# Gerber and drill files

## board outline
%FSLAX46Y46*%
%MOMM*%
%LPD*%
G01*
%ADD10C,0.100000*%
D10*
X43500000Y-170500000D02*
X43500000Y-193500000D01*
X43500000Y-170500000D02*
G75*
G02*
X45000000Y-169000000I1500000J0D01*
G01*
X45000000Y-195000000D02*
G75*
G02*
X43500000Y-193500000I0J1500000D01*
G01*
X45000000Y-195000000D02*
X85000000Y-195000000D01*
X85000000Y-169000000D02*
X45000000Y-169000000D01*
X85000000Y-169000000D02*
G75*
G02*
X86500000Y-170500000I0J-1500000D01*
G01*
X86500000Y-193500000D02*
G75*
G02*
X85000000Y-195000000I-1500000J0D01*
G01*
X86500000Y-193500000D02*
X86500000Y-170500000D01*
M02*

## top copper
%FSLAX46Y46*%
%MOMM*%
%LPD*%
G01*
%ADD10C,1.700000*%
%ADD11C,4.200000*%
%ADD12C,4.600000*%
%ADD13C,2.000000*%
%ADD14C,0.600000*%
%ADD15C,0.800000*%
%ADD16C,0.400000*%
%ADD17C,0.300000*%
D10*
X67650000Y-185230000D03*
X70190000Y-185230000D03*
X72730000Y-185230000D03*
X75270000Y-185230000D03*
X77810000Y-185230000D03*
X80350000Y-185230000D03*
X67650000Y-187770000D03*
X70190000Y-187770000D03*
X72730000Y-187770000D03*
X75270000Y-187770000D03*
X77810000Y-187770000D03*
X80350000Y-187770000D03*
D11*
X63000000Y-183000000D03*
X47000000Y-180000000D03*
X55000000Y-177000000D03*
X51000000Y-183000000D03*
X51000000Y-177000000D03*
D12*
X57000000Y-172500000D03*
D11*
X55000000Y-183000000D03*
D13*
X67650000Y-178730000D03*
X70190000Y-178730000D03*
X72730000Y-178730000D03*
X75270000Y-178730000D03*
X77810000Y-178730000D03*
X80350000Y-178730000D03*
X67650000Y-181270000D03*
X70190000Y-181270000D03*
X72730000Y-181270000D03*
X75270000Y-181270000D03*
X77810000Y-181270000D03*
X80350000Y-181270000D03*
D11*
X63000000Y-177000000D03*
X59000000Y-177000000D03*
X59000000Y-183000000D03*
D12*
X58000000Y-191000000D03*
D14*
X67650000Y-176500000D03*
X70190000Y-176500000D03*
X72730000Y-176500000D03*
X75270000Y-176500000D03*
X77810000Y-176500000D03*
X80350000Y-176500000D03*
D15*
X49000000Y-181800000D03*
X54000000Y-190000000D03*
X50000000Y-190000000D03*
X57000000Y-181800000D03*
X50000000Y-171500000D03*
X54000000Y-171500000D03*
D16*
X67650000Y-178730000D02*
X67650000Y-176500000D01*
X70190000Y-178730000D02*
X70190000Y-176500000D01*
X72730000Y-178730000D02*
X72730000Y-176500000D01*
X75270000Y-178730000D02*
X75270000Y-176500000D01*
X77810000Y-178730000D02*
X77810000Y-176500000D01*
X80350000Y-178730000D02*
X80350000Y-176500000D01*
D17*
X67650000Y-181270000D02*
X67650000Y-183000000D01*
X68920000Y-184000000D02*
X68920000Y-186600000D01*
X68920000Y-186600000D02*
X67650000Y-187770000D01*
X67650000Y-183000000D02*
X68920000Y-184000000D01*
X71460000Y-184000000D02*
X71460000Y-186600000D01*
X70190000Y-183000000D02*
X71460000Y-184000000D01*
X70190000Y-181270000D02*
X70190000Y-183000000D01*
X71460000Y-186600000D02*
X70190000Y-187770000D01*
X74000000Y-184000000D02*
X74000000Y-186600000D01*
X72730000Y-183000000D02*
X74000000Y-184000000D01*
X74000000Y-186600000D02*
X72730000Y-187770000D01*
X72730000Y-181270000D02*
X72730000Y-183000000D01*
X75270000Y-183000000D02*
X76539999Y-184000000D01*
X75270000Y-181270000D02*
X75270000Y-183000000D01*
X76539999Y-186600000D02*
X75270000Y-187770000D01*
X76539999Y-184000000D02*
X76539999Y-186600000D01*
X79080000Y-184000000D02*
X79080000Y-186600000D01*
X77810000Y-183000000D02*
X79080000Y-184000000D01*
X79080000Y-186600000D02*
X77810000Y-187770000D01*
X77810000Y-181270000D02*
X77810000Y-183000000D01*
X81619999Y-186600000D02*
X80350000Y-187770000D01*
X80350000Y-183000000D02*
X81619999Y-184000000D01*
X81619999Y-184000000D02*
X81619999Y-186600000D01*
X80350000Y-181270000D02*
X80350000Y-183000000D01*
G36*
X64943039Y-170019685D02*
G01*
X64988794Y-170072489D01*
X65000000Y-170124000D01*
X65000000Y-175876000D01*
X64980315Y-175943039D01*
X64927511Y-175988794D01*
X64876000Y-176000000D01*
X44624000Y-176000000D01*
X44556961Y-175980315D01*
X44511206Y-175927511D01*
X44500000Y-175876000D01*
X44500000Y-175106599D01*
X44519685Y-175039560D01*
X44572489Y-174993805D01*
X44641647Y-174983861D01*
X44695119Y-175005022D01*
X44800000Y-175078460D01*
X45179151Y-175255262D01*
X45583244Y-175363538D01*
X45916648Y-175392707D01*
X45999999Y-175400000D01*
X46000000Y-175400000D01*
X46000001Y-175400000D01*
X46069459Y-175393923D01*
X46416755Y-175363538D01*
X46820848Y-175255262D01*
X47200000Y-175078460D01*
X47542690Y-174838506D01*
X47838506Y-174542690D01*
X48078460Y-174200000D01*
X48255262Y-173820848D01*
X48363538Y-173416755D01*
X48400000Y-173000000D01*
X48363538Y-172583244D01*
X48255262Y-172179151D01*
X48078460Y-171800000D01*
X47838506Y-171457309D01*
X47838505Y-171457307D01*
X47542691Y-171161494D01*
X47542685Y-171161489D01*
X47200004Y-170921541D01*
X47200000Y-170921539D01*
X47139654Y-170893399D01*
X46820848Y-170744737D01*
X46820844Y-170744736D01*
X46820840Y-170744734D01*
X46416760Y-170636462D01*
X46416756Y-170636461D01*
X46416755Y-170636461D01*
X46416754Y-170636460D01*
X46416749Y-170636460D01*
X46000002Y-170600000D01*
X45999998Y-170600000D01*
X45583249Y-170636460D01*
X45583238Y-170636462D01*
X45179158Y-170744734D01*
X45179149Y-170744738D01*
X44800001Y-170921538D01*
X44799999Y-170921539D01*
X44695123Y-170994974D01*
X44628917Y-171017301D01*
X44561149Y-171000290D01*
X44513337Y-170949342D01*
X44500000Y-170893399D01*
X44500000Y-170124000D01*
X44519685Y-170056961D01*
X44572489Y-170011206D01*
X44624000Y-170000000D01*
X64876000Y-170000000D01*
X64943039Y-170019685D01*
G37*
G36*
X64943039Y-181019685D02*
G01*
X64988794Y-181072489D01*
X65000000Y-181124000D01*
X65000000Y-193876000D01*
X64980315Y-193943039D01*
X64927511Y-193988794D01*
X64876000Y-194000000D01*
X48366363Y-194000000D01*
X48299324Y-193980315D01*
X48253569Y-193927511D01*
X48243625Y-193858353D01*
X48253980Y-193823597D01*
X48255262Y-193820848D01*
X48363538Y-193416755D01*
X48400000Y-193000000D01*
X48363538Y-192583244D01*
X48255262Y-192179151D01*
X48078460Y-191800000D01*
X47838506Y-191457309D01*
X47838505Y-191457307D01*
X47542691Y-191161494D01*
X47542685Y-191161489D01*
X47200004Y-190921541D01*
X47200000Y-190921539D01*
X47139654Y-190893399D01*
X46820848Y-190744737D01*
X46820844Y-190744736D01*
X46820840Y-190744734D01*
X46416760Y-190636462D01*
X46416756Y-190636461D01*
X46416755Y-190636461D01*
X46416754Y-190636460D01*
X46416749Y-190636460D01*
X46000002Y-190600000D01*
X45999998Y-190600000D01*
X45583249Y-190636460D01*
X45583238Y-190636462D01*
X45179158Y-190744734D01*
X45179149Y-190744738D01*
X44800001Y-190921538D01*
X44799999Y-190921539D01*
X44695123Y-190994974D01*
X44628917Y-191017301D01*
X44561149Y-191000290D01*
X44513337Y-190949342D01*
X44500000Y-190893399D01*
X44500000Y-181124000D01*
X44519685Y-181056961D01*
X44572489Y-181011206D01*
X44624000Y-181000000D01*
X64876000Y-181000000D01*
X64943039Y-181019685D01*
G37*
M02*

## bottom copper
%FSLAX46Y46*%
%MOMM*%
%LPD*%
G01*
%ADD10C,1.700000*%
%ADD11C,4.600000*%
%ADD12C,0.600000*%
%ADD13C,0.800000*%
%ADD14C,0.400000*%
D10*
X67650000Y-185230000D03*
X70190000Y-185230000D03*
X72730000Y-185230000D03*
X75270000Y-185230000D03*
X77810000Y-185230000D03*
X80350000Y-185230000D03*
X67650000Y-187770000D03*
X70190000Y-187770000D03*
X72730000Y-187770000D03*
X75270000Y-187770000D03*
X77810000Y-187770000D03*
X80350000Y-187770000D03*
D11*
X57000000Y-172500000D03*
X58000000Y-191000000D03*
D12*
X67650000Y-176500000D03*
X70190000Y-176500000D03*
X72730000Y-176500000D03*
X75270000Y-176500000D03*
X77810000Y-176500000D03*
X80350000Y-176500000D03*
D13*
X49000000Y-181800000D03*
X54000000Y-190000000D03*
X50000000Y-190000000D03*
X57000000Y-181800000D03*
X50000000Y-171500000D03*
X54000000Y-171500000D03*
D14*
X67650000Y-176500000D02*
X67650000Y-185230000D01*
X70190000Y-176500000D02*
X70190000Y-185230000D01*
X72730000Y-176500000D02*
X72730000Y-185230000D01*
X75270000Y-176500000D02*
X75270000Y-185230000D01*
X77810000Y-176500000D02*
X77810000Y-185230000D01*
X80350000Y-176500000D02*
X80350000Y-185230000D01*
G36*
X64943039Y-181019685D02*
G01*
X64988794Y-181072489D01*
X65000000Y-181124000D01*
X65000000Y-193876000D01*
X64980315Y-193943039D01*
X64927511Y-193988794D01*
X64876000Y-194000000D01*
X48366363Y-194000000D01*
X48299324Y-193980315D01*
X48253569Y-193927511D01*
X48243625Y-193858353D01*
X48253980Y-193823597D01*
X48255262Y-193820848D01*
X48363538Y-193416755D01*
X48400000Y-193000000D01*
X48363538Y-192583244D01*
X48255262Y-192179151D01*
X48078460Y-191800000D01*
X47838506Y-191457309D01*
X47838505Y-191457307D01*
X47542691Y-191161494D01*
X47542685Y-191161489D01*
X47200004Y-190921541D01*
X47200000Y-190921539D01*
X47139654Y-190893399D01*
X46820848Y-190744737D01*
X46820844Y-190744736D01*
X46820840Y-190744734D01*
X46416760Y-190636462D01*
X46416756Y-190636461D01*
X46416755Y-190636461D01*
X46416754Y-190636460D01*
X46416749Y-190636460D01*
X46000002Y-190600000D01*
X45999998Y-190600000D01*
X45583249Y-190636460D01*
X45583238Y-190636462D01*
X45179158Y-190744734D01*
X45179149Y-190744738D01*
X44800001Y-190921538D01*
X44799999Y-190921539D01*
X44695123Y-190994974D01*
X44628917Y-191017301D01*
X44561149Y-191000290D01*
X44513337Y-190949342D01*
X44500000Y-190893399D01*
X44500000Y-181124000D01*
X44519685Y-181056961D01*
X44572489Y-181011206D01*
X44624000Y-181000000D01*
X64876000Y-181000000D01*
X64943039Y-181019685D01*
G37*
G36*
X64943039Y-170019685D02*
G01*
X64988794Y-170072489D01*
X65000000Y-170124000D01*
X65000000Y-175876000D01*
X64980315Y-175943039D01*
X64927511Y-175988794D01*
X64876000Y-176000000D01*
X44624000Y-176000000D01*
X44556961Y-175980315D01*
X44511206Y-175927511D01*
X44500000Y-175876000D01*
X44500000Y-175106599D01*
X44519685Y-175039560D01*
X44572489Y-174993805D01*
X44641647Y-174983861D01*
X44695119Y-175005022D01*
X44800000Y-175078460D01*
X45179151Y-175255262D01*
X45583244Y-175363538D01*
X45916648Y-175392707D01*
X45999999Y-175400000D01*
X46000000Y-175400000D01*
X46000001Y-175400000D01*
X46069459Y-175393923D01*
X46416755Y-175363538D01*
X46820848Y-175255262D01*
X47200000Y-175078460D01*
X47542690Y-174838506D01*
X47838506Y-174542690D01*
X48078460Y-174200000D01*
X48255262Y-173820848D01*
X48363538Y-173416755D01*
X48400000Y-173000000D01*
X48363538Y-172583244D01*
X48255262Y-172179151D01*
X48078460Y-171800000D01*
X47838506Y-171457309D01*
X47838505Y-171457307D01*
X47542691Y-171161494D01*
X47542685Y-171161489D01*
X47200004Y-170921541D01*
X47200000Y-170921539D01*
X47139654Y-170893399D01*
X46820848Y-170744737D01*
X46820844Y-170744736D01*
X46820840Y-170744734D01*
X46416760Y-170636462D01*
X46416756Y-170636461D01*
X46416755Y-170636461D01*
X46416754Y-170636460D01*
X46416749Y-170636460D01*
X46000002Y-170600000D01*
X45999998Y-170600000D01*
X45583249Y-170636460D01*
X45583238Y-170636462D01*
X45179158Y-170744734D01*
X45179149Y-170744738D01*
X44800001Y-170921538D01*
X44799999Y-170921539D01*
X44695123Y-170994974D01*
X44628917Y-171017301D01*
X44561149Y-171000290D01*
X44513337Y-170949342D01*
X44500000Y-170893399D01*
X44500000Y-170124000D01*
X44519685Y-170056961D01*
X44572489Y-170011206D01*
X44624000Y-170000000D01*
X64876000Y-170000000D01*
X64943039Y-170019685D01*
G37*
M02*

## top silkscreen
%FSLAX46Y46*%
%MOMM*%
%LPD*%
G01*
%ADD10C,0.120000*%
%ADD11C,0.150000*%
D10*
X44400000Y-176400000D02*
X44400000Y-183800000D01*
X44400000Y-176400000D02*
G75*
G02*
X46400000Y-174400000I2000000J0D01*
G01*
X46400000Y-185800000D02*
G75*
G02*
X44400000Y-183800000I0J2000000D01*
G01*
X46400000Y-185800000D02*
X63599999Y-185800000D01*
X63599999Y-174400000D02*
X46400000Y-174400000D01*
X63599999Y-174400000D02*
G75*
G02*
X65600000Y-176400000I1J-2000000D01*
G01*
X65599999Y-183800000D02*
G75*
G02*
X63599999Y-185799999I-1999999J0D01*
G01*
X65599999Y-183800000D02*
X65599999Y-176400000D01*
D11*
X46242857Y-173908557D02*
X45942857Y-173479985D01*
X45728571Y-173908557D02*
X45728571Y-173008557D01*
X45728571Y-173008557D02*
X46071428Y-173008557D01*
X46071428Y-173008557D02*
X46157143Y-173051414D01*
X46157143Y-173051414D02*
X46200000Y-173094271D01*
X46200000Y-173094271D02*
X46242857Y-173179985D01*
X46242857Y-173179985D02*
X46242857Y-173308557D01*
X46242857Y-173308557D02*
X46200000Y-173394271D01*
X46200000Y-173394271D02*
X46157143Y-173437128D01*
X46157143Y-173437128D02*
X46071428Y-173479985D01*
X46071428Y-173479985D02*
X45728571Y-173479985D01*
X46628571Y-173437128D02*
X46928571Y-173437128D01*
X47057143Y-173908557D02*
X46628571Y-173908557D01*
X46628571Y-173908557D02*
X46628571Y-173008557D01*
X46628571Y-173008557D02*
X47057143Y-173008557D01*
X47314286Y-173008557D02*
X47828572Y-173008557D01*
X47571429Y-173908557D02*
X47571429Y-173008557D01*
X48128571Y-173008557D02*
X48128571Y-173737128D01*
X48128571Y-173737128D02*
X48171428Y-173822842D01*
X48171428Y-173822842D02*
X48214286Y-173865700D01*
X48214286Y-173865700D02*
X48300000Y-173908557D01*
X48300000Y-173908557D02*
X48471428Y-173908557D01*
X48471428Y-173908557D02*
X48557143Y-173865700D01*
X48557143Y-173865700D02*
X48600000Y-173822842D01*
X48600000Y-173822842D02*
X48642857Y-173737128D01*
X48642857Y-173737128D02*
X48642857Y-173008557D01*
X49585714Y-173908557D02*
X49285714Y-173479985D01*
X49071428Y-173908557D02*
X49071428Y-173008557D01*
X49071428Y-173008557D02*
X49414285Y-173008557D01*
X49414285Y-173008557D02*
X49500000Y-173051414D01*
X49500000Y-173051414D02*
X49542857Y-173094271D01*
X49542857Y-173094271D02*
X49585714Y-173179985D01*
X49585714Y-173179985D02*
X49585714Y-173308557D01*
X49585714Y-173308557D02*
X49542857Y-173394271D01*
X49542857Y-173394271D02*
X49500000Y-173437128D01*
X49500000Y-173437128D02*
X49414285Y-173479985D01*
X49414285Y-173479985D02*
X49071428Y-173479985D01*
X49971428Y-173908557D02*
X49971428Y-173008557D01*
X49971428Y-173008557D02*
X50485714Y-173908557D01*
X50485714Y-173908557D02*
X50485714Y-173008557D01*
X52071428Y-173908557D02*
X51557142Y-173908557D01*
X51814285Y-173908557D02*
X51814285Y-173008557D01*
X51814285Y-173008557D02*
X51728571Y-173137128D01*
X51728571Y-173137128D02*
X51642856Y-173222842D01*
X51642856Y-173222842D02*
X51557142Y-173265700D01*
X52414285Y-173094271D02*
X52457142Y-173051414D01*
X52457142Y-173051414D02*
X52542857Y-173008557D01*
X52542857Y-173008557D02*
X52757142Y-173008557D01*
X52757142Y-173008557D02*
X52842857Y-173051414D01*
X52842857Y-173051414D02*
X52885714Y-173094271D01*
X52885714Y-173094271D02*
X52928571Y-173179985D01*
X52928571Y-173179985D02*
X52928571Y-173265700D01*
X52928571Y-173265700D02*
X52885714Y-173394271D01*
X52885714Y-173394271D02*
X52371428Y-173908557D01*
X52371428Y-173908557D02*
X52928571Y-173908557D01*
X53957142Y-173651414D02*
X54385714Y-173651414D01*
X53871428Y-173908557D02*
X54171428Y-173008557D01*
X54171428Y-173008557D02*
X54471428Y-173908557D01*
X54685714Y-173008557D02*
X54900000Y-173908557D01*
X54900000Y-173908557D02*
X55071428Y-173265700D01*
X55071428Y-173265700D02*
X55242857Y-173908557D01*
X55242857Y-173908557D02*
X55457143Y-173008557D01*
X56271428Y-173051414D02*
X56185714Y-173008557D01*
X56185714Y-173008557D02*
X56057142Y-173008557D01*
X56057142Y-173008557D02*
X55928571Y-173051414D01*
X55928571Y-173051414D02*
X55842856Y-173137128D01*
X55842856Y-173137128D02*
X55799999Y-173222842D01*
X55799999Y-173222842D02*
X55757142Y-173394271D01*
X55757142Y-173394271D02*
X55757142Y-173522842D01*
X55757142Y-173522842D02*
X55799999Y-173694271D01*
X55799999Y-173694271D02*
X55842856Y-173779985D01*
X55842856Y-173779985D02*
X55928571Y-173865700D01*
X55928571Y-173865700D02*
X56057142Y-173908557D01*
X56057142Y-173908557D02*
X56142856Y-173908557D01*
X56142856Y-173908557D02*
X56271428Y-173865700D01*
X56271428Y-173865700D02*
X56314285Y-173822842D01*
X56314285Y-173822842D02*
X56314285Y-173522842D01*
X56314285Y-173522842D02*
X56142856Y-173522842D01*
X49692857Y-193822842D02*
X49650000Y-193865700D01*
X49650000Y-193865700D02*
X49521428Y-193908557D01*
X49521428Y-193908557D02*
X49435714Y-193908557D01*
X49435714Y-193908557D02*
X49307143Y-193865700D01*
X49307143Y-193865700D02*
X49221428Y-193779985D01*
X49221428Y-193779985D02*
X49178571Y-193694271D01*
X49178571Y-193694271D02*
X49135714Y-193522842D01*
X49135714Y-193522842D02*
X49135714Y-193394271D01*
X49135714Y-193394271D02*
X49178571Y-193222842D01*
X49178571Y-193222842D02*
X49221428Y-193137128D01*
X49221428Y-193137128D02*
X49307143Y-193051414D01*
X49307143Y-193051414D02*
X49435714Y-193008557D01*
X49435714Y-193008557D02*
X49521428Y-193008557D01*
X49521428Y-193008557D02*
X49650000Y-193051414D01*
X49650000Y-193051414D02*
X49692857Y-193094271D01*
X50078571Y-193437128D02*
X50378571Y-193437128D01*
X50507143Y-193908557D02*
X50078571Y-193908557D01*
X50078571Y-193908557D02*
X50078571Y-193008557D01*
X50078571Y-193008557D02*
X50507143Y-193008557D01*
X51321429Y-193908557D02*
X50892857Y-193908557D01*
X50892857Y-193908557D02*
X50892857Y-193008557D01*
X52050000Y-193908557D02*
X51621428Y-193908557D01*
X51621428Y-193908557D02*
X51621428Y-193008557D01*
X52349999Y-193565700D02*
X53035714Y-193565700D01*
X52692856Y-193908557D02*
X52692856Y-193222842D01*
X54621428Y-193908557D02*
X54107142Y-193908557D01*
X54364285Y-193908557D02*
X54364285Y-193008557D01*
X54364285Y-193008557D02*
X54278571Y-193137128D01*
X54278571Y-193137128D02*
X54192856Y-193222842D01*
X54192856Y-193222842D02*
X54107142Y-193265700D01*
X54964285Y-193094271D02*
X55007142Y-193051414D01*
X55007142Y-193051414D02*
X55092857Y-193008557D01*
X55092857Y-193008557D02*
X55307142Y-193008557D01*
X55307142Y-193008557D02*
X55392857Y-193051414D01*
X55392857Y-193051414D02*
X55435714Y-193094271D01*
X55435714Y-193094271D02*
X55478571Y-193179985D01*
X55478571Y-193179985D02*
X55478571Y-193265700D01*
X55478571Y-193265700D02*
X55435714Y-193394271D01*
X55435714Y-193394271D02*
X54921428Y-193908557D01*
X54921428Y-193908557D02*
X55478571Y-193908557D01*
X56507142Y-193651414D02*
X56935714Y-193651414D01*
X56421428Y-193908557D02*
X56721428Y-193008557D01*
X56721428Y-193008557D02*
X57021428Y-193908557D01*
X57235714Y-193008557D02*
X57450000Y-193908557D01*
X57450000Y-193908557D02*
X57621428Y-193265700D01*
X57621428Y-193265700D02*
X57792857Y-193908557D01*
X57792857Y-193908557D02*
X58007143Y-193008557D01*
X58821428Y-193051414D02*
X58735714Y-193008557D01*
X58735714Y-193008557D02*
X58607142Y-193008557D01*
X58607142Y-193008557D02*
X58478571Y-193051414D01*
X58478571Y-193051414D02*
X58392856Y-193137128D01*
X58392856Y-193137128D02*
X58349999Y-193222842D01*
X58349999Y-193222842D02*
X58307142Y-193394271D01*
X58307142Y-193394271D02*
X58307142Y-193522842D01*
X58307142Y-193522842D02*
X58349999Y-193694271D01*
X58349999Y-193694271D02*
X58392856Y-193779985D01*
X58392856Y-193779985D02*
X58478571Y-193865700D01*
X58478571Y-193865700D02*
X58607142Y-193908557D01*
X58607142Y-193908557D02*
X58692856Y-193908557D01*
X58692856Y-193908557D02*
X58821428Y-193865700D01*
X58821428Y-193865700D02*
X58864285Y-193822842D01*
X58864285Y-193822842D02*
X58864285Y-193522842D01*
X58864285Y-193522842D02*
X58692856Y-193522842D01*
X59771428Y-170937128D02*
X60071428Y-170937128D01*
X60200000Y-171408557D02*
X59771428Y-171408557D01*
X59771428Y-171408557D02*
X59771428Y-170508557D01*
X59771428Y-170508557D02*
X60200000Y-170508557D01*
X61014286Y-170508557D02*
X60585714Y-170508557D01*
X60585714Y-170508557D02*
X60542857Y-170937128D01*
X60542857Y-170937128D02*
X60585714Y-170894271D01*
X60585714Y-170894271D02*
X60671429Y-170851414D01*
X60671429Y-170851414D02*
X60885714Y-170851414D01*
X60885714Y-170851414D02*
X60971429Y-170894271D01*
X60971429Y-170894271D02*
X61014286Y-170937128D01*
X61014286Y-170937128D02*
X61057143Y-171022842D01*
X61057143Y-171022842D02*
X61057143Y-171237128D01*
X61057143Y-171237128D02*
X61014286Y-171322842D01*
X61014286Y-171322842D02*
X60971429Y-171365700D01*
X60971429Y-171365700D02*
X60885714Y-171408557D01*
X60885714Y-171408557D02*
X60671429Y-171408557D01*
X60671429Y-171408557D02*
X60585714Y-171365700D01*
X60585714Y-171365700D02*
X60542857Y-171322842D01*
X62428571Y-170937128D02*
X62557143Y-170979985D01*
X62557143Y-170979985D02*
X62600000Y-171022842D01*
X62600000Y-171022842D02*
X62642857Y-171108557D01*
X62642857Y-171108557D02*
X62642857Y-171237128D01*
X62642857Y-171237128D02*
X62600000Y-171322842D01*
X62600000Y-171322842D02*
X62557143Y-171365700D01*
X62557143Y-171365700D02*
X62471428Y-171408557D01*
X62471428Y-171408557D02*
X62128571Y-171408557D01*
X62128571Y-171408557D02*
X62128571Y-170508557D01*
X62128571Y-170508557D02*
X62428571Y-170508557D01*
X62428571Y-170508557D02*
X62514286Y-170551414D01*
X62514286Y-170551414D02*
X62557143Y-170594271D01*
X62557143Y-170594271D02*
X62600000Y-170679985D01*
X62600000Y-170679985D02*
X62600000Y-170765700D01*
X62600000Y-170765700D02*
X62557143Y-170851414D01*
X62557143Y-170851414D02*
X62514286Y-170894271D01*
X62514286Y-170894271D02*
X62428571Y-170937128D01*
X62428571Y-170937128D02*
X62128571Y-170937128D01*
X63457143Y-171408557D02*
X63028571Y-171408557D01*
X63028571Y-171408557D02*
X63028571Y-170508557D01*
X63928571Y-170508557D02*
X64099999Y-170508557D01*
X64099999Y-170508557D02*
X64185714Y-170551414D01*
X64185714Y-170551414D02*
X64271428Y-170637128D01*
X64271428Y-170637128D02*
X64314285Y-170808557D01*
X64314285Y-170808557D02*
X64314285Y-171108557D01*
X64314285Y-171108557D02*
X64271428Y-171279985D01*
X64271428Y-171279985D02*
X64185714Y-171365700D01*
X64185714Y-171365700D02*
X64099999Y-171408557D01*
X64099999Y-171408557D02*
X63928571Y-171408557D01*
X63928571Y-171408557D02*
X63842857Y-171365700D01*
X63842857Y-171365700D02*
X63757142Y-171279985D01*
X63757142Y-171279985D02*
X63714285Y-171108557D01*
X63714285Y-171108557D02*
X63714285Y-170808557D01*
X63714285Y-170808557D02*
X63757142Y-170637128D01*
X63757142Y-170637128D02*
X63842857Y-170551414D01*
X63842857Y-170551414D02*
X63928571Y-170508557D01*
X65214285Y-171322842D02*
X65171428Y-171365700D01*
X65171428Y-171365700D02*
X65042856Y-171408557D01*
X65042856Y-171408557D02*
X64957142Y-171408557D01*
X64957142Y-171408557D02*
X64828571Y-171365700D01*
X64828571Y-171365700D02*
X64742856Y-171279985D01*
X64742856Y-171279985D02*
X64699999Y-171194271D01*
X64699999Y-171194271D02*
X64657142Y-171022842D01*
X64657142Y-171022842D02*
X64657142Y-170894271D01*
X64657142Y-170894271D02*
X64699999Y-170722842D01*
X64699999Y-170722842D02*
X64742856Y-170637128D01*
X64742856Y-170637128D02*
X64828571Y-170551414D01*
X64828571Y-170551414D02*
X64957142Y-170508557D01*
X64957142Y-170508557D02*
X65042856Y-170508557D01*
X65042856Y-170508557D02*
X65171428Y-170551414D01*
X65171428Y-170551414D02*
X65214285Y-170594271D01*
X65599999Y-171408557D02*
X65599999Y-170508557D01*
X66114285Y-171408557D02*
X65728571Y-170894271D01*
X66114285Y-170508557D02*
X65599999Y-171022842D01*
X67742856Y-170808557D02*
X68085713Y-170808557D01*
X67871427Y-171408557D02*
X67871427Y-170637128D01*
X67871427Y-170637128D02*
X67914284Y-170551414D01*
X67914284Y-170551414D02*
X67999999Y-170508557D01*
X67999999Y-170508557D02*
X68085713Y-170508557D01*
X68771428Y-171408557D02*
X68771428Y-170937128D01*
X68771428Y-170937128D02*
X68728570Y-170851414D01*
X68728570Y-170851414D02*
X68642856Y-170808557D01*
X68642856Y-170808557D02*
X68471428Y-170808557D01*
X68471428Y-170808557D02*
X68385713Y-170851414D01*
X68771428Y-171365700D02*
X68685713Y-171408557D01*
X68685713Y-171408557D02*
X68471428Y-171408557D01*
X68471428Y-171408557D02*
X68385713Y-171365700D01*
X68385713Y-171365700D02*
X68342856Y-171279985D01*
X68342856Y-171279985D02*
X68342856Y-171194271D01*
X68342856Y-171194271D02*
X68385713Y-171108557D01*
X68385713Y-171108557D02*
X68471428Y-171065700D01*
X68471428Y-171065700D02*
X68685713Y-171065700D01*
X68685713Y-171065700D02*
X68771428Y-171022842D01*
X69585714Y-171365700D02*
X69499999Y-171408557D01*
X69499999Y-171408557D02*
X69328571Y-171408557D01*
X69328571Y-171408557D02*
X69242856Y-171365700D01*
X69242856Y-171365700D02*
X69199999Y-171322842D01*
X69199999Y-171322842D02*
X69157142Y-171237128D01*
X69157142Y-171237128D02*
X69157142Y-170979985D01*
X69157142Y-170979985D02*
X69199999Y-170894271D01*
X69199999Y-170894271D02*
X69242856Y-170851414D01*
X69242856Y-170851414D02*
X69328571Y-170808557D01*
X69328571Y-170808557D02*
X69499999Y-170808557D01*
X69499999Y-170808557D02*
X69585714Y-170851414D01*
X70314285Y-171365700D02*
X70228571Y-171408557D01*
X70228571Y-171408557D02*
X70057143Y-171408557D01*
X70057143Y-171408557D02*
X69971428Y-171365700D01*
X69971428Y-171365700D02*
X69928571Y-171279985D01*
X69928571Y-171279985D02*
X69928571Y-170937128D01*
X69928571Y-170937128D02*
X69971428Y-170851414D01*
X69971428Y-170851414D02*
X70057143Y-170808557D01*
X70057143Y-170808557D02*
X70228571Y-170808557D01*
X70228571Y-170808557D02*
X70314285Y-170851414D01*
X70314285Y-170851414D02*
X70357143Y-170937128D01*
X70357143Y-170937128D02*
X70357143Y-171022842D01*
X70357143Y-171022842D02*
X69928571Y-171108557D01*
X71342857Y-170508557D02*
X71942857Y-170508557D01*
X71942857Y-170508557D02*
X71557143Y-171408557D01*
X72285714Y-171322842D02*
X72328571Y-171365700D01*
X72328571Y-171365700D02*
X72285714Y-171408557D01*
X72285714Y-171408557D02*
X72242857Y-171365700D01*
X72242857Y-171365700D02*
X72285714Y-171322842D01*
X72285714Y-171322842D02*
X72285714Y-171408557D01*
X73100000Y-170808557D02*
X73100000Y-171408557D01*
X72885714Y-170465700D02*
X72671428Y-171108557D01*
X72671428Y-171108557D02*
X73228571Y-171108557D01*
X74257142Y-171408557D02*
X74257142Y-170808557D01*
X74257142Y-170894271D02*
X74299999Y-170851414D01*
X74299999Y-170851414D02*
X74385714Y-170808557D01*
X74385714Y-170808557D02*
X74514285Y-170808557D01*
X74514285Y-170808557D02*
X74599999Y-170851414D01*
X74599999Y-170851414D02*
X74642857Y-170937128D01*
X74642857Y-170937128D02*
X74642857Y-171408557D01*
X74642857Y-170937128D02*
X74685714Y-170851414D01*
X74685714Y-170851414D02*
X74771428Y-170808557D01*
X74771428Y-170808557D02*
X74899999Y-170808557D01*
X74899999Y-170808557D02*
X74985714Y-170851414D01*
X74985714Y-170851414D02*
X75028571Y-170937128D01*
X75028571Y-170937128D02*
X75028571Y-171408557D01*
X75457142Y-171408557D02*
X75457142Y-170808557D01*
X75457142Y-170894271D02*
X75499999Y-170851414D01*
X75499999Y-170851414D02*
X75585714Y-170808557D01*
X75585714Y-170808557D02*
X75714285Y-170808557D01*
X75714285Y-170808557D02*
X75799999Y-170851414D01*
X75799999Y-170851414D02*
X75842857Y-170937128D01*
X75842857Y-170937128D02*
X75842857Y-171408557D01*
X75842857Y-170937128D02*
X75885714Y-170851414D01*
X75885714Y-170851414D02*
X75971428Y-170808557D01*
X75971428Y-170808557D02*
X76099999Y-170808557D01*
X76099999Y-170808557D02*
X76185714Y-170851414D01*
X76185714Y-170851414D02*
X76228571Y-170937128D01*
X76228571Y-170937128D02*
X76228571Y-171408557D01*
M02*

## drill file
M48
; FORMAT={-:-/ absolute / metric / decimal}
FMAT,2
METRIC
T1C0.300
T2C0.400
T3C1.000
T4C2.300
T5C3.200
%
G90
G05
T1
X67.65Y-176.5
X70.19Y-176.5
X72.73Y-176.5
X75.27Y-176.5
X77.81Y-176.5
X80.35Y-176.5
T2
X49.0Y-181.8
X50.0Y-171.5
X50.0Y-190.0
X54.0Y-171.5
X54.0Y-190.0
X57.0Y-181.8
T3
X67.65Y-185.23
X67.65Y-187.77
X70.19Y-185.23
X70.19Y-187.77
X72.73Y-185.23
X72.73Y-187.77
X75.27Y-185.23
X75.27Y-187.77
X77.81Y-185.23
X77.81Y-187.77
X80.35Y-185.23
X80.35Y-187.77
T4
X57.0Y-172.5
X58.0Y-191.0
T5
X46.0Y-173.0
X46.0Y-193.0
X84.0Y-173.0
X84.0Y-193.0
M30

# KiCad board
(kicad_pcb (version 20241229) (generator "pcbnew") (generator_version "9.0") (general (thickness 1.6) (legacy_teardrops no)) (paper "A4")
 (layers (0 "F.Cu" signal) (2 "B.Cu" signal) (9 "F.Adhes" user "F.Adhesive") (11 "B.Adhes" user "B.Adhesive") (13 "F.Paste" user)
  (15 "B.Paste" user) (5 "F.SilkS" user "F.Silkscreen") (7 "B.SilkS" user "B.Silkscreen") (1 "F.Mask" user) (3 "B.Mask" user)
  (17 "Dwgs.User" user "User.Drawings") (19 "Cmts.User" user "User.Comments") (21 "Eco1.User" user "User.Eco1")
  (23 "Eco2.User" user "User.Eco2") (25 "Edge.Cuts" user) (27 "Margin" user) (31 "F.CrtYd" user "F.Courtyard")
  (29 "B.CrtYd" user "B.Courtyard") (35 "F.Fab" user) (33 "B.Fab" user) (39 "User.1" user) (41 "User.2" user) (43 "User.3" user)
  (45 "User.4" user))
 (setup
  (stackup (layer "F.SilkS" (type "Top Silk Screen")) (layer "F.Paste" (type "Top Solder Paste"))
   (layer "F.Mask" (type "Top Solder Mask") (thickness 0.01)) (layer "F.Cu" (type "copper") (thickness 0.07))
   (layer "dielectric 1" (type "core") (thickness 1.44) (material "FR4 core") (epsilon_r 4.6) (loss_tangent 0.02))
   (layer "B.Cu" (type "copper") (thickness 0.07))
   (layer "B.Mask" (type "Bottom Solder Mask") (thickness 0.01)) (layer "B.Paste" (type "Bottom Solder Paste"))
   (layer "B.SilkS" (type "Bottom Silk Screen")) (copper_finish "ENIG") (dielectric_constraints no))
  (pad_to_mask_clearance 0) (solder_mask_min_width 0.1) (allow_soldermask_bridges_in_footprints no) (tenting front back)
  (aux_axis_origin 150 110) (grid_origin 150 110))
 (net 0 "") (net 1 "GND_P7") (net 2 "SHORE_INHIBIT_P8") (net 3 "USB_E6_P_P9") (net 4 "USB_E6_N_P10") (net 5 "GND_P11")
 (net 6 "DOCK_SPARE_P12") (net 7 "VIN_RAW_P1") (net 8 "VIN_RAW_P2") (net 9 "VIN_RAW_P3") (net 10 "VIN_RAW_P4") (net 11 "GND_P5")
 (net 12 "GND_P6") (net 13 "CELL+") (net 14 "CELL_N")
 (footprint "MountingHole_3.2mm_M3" (layer "F.Cu") (at 84 193)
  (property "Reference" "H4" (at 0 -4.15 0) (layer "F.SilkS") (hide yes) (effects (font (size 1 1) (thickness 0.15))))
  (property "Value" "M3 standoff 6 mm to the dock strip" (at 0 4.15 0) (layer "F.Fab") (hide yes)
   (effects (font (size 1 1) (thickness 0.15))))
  (pad "" np_thru_hole circle (at 0 0) (size 3.2 3.2) (drill 3.2) (layers "*.Cu" "*.Mask")))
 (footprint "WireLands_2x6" (layer "F.Cu") (at 74 186.5)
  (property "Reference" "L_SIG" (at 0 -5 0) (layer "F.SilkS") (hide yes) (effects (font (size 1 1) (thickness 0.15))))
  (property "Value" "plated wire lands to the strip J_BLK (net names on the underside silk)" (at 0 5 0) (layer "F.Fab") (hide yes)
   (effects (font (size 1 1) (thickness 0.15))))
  (pad "1" thru_hole circle (at -6.35 -1.27) (size 1.7 1.7) (drill 1) (layers "*.Cu" "*.Mask") (remove_unused_layers no) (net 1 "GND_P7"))
  (pad "2" thru_hole circle (at -3.81 -1.27) (size 1.7 1.7) (drill 1) (layers "*.Cu" "*.Mask") (remove_unused_layers no)
   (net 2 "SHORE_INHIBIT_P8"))
  (pad "3" thru_hole circle (at -1.27 -1.27) (size 1.7 1.7) (drill 1) (layers "*.Cu" "*.Mask") (remove_unused_layers no)
   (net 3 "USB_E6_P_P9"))
  (pad "4" thru_hole circle (at 1.27 -1.27) (size 1.7 1.7) (drill 1) (layers "*.Cu" "*.Mask") (remove_unused_layers no)
   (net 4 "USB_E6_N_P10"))
  (pad "5" thru_hole circle (at 3.81 -1.27) (size 1.7 1.7) (drill 1) (layers "*.Cu" "*.Mask") (remove_unused_layers no) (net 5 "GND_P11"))
  (pad "6" thru_hole circle (at 6.35 -1.27) (size 1.7 1.7) (drill 1) (layers "*.Cu" "*.Mask") (remove_unused_layers no)
   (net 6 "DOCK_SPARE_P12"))
  (pad "7" thru_hole circle (at -6.35 1.27) (size 1.7 1.7) (drill 1) (layers "*.Cu" "*.Mask") (remove_unused_layers no) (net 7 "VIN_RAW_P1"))
  (pad "8" thru_hole circle (at -3.81 1.27) (size 1.7 1.7) (drill 1) (layers "*.Cu" "*.Mask") (remove_unused_layers no) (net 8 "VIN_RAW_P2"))
  (pad "9" thru_hole circle (at -1.27 1.27) (size 1.7 1.7) (drill 1) (layers "*.Cu" "*.Mask") (remove_unused_layers no) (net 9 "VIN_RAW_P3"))
  (pad "10" thru_hole circle (at 1.27 1.27) (size 1.7 1.7) (drill 1) (layers "*.Cu" "*.Mask") (remove_unused_layers no)
   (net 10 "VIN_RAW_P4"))
  (pad "11" thru_hole circle (at 3.81 1.27) (size 1.7 1.7) (drill 1) (layers "*.Cu" "*.Mask") (remove_unused_layers no) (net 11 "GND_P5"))
  (pad "12" thru_hole circle (at 6.35 1.27) (size 1.7 1.7) (drill 1) (layers "*.Cu" "*.Mask") (remove_unused_layers no) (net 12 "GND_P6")))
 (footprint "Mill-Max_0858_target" (layer "F.Cu") (at 63 183)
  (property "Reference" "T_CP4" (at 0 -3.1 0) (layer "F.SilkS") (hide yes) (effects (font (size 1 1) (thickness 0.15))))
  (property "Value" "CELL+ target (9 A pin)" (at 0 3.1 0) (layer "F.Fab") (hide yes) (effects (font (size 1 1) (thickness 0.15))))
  (pad "1" smd circle (at 0 0) (size 4.2 4.2) (layers "F.Cu" "F.Mask") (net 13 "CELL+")))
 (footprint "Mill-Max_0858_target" (layer "F.Cu") (at 47 180)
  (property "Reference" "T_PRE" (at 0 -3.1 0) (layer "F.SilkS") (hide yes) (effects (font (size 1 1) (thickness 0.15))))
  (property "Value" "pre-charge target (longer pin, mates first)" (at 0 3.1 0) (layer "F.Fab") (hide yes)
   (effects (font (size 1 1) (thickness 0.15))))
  (pad "1" smd circle (at 0 0) (size 4.2 4.2) (layers "F.Cu" "F.Mask") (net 13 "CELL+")))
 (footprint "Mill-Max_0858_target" (layer "F.Cu") (at 55 177)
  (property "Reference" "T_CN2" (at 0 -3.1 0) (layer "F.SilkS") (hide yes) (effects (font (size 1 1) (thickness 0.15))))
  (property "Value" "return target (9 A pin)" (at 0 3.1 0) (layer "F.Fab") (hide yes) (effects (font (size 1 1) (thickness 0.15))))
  (pad "1" smd circle (at 0 0) (size 4.2 4.2) (layers "F.Cu" "F.Mask") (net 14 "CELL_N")))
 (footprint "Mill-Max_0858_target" (layer "F.Cu") (at 51 183)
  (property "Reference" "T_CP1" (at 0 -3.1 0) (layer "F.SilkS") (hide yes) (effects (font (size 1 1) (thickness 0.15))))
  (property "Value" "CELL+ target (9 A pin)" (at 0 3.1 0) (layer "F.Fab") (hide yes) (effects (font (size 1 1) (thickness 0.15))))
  (pad "1" smd circle (at 0 0) (size 4.2 4.2) (layers "F.Cu" "F.Mask") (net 13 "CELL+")))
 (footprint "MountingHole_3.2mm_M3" (layer "F.Cu") (at 84 173)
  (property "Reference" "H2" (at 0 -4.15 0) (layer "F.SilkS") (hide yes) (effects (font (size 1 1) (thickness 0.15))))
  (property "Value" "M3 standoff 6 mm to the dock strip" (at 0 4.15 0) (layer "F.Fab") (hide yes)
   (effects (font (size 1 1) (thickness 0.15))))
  (pad "" np_thru_hole circle (at 0 0) (size 3.2 3.2) (drill 3.2) (layers "*.Cu" "*.Mask")))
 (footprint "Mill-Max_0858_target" (layer "F.Cu") (at 51 177)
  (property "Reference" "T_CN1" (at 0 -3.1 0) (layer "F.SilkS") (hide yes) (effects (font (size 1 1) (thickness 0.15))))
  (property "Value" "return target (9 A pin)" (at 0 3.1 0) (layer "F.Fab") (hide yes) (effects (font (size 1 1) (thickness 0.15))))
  (pad "1" smd circle (at 0 0) (size 4.2 4.2) (layers "F.Cu" "F.Mask") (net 14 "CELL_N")))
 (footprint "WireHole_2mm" (layer "F.Cu") (at 57 172.5)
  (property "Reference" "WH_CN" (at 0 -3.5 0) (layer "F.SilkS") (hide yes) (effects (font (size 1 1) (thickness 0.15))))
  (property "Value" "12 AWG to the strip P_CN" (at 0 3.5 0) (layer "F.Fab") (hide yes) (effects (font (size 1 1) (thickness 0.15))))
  (pad "1" thru_hole circle (at 0 0) (size 4.6 4.6) (drill 2.3) (layers "*.Cu" "*.Mask") (remove_unused_layers no) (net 14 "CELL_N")))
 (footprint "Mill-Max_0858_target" (layer "F.Cu") (at 55 183)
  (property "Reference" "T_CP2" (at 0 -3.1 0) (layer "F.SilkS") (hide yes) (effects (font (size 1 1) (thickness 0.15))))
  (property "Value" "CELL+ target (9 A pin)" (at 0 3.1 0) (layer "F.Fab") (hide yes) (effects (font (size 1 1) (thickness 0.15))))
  (pad "1" smd circle (at 0 0) (size 4.2 4.2) (layers "F.Cu" "F.Mask") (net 13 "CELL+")))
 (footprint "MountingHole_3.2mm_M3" (layer "F.Cu") (at 46 173)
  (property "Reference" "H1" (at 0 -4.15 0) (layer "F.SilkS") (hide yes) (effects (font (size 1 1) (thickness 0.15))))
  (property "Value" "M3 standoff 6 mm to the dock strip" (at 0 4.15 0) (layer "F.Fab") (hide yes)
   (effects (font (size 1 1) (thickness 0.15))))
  (pad "" np_thru_hole circle (at 0 0) (size 3.2 3.2) (drill 3.2) (layers "*.Cu" "*.Mask")))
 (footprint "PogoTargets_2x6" (layer "F.Cu") (at 74 180)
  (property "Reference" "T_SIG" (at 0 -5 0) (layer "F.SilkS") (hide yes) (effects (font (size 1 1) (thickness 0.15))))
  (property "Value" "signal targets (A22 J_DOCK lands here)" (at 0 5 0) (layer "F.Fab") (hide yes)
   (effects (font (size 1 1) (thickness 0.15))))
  (pad "1" smd circle (at -6.35 -1.27) (size 2 2) (layers "F.Cu" "F.Mask") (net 1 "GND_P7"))
  (pad "2" smd circle (at -3.81 -1.27) (size 2 2) (layers "F.Cu" "F.Mask") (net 2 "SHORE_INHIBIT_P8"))
  (pad "3" smd circle (at -1.27 -1.27) (size 2 2) (layers "F.Cu" "F.Mask") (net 3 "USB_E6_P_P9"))
  (pad "4" smd circle (at 1.27 -1.27) (size 2 2) (layers "F.Cu" "F.Mask") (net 4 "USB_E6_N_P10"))
  (pad "5" smd circle (at 3.81 -1.27) (size 2 2) (layers "F.Cu" "F.Mask") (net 5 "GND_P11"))
  (pad "6" smd circle (at 6.35 -1.27) (size 2 2) (layers "F.Cu" "F.Mask") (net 6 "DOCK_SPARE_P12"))
  (pad "7" smd circle (at -6.35 1.27) (size 2 2) (layers "F.Cu" "F.Mask") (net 7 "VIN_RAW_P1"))
  (pad "8" smd circle (at -3.81 1.27) (size 2 2) (layers "F.Cu" "F.Mask") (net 8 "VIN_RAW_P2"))
  (pad "9" smd circle (at -1.27 1.27) (size 2 2) (layers "F.Cu" "F.Mask") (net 9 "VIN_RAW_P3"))
  (pad "10" smd circle (at 1.27 1.27) (size 2 2) (layers "F.Cu" "F.Mask") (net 10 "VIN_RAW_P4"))
  (pad "11" smd circle (at 3.81 1.27) (size 2 2) (layers "F.Cu" "F.Mask") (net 11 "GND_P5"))
  (pad "12" smd circle (at 6.35 1.27) (size 2 2) (layers "F.Cu" "F.Mask") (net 12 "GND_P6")))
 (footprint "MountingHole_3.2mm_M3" (layer "F.Cu") (at 46 193)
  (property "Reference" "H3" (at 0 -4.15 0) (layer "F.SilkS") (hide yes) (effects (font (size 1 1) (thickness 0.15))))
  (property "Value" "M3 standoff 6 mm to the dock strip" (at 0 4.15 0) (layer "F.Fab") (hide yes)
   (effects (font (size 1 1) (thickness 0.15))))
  (pad "" np_thru_hole circle (at 0 0) (size 3.2 3.2) (drill 3.2) (layers "*.Cu" "*.Mask")))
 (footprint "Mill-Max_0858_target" (layer "F.Cu") (at 63 177)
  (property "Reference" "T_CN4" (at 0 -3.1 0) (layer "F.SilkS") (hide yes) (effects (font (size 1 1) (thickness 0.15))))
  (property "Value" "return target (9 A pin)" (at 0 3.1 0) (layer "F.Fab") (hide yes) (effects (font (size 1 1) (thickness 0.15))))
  (pad "1" smd circle (at 0 0) (size 4.2 4.2) (layers "F.Cu" "F.Mask") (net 14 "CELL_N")))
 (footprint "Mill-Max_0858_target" (layer "F.Cu") (at 59 177)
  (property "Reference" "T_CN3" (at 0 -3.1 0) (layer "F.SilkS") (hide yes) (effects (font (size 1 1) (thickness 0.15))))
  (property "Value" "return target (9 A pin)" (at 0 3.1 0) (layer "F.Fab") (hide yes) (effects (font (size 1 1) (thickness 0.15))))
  (pad "1" smd circle (at 0 0) (size 4.2 4.2) (layers "F.Cu" "F.Mask") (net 14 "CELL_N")))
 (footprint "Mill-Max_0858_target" (layer "F.Cu") (at 59 183)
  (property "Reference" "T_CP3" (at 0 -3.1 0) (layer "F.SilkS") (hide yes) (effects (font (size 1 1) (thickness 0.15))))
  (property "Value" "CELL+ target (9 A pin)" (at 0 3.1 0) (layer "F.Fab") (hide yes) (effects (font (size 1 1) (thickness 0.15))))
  (pad "1" smd circle (at 0 0) (size 4.2 4.2) (layers "F.Cu" "F.Mask") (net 13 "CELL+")))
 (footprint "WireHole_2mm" (layer "F.Cu") (at 58 191)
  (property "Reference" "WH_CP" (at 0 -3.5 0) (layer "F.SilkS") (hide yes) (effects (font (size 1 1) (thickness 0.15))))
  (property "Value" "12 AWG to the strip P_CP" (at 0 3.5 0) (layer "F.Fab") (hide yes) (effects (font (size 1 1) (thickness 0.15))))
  (pad "1" thru_hole circle (at 0 0) (size 4.6 4.6) (drill 2.3) (layers "*.Cu" "*.Mask") (remove_unused_layers no) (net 13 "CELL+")))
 (gr_line (start 44.4 176.4) (end 44.4 183.8) (stroke (width 0.12) (type default)) (layer "F.SilkS"))
 (gr_arc (start 44.4 176.4) (mid 44.985786 174.985786) (end 46.4 174.4) (stroke (width 0.12) (type default)) (layer "F.SilkS"))
 (gr_arc (start 46.4 185.8) (mid 44.985786 185.214214) (end 44.4 183.8) (stroke (width 0.12) (type default)) (layer "F.SilkS"))
 (gr_line (start 46.4 185.8) (end 63.599999 185.8) (stroke (width 0.12) (type default)) (layer "F.SilkS"))
 (gr_line (start 63.599999 174.4) (end 46.4 174.4) (stroke (width 0.12) (type default)) (layer "F.SilkS"))
 (gr_arc (start 63.599999 174.4) (mid 65.014213 174.985786) (end 65.599999 176.4) (stroke (width 0.12) (type default)) (layer "F.SilkS"))
 (gr_arc (start 65.599999 183.8) (mid 65.014213 185.214213) (end 63.599999 185.8) (stroke (width 0.12) (type default)) (layer "F.SilkS"))
 (gr_line (start 65.599999 183.8) (end 65.599999 176.4) (stroke (width 0.12) (type default)) (layer "F.SilkS"))
 (gr_line (start 43.5 170.5) (end 43.5 193.5) (stroke (width 0.1) (type default)) (layer "Edge.Cuts"))
 (gr_arc (start 43.5 170.5) (mid 43.93934 169.43934) (end 45 169) (stroke (width 0.1) (type default)) (layer "Edge.Cuts"))
 (gr_arc (start 45 195) (mid 43.93934 194.56066) (end 43.5 193.5) (stroke (width 0.1) (type default)) (layer "Edge.Cuts"))
 (gr_line (start 45 195) (end 85 195) (stroke (width 0.1) (type default)) (layer "Edge.Cuts"))
 (gr_line (start 85 169) (end 45 169) (stroke (width 0.1) (type default)) (layer "Edge.Cuts"))
 (gr_arc (start 85 169) (mid 86.06066 169.43934) (end 86.5 170.5) (stroke (width 0.1) (type default)) (layer "Edge.Cuts"))
 (gr_arc (start 86.5 193.5) (mid 86.06066 194.56066) (end 85 195) (stroke (width 0.1) (type default)) (layer "Edge.Cuts"))
 (gr_line (start 86.5 193.5) (end 86.5 170.5) (stroke (width 0.1) (type default)) (layer "Edge.Cuts"))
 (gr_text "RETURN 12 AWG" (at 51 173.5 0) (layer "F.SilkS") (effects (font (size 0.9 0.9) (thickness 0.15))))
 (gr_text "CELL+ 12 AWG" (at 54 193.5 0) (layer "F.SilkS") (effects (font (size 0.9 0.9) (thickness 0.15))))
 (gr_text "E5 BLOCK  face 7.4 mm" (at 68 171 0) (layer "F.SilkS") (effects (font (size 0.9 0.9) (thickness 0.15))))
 (segment (start 67.65 178.73) (end 67.65 176.5) (width 0.4) (layer "F.Cu") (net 1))
 (via (at 67.65 176.5) (size 0.6) (drill 0.3) (layers "F.Cu" "B.Cu") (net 1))
 (segment (start 67.65 176.5) (end 67.65 185.23) (width 0.4) (layer "B.Cu") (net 1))
 (segment (start 70.19 178.73) (end 70.19 176.5) (width 0.4) (layer "F.Cu") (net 2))
 (via (at 70.19 176.5) (size 0.6) (drill 0.3) (layers "F.Cu" "B.Cu") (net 2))
 (segment (start 70.19 176.5) (end 70.19 185.23) (width 0.4) (layer "B.Cu") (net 2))
 (segment (start 72.73 178.73) (end 72.73 176.5) (width 0.4) (layer "F.Cu") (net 3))
 (via (at 72.73 176.5) (size 0.6) (drill 0.3) (layers "F.Cu" "B.Cu") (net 3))
 (segment (start 72.73 176.5) (end 72.73 185.23) (width 0.4) (layer "B.Cu") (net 3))
 (segment (start 75.27 178.73) (end 75.27 176.5) (width 0.4) (layer "F.Cu") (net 4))
 (via (at 75.27 176.5) (size 0.6) (drill 0.3) (layers "F.Cu" "B.Cu") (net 4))
 (segment (start 75.27 176.5) (end 75.27 185.23) (width 0.4) (layer "B.Cu") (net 4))
 (segment (start 77.81 178.73) (end 77.81 176.5) (width 0.4) (layer "F.Cu") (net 5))
 (via (at 77.81 176.5) (size 0.6) (drill 0.3) (layers "F.Cu" "B.Cu") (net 5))
 (segment (start 77.81 176.5) (end 77.81 185.23) (width 0.4) (layer "B.Cu") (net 5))
 (segment (start 80.35 178.73) (end 80.35 176.5) (width 0.4) (layer "F.Cu") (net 6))
 (via (at 80.35 176.5) (size 0.6) (drill 0.3) (layers "F.Cu" "B.Cu") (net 6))
 (segment (start 80.35 176.5) (end 80.35 185.23) (width 0.4) (layer "B.Cu") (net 6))
 (segment (start 67.65 181.27) (end 67.65 183) (width 0.3) (layer "F.Cu") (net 7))
 (segment (start 68.92 184) (end 68.92 186.6) (width 0.3) (layer "F.Cu") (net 7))
 (segment (start 68.92 186.6) (end 67.65 187.77) (width 0.3) (layer "F.Cu") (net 7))
 (segment (start 67.65 183) (end 68.92 184) (width 0.3) (layer "F.Cu") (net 7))
 (segment (start 71.46 184) (end 71.46 186.6) (width 0.3) (layer "F.Cu") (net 8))
 (segment (start 70.19 183) (end 71.46 184) (width 0.3) (layer "F.Cu") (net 8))
 (segment (start 70.19 181.27) (end 70.19 183) (width 0.3) (layer "F.Cu") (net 8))
 (segment (start 71.46 186.6) (end 70.19 187.77) (width 0.3) (layer "F.Cu") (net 8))
 (segment (start 74 184) (end 74 186.6) (width 0.3) (layer "F.Cu") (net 9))
 (segment (start 72.73 183) (end 74 184) (width 0.3) (layer "F.Cu") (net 9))
 (segment (start 74 186.6) (end 72.73 187.77) (width 0.3) (layer "F.Cu") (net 9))
 (segment (start 72.73 181.27) (end 72.73 183) (width 0.3) (layer "F.Cu") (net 9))
 (segment (start 75.27 183) (end 76.539999 184) (width 0.3) (layer "F.Cu") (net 10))
 (segment (start 75.27 181.27) (end 75.27 183) (width 0.3) (layer "F.Cu") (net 10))
 (segment (start 76.539999 186.6) (end 75.27 187.77) (width 0.3) (layer "F.Cu") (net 10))
 (segment (start 76.539999 184) (end 76.539999 186.6) (width 0.3) (layer "F.Cu") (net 10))
 (segment (start 79.08 184) (end 79.08 186.6) (width 0.3) (layer "F.Cu") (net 11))
 (segment (start 77.81 183) (end 79.08 184) (width 0.3) (layer "F.Cu") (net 11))
 (segment (start 79.08 186.6) (end 77.81 187.77) (width 0.3) (layer "F.Cu") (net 11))
 (segment (start 77.81 181.27) (end 77.81 183) (width 0.3) (layer "F.Cu") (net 11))
 (segment (start 81.619999 186.6) (end 80.35 187.77) (width 0.3) (layer "F.Cu") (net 12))
 (segment (start 80.35 183) (end 81.619999 184) (width 0.3) (layer "F.Cu") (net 12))
 (segment (start 81.619999 184) (end 81.619999 186.6) (width 0.3) (layer "F.Cu") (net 12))
 (segment (start 80.35 181.27) (end 80.35 183) (width 0.3) (layer "F.Cu") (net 12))
 (via (at 49 181.8) (size 0.8) (drill 0.4) (layers "F.Cu" "B.Cu") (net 13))
 (via (at 54 190) (size 0.8) (drill 0.4) (layers "F.Cu" "B.Cu") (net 13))
 (via (at 50 190) (size 0.8) (drill 0.4) (layers "F.Cu" "B.Cu") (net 13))
 (via (at 57 181.8) (size 0.8) (drill 0.4) (layers "F.Cu" "B.Cu") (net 13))
 (via (at 50 171.5) (size 0.8) (drill 0.4) (layers "F.Cu" "B.Cu") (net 14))
 (via (at 54 171.5) (size 0.8) (drill 0.4) (layers "F.Cu" "B.Cu") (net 14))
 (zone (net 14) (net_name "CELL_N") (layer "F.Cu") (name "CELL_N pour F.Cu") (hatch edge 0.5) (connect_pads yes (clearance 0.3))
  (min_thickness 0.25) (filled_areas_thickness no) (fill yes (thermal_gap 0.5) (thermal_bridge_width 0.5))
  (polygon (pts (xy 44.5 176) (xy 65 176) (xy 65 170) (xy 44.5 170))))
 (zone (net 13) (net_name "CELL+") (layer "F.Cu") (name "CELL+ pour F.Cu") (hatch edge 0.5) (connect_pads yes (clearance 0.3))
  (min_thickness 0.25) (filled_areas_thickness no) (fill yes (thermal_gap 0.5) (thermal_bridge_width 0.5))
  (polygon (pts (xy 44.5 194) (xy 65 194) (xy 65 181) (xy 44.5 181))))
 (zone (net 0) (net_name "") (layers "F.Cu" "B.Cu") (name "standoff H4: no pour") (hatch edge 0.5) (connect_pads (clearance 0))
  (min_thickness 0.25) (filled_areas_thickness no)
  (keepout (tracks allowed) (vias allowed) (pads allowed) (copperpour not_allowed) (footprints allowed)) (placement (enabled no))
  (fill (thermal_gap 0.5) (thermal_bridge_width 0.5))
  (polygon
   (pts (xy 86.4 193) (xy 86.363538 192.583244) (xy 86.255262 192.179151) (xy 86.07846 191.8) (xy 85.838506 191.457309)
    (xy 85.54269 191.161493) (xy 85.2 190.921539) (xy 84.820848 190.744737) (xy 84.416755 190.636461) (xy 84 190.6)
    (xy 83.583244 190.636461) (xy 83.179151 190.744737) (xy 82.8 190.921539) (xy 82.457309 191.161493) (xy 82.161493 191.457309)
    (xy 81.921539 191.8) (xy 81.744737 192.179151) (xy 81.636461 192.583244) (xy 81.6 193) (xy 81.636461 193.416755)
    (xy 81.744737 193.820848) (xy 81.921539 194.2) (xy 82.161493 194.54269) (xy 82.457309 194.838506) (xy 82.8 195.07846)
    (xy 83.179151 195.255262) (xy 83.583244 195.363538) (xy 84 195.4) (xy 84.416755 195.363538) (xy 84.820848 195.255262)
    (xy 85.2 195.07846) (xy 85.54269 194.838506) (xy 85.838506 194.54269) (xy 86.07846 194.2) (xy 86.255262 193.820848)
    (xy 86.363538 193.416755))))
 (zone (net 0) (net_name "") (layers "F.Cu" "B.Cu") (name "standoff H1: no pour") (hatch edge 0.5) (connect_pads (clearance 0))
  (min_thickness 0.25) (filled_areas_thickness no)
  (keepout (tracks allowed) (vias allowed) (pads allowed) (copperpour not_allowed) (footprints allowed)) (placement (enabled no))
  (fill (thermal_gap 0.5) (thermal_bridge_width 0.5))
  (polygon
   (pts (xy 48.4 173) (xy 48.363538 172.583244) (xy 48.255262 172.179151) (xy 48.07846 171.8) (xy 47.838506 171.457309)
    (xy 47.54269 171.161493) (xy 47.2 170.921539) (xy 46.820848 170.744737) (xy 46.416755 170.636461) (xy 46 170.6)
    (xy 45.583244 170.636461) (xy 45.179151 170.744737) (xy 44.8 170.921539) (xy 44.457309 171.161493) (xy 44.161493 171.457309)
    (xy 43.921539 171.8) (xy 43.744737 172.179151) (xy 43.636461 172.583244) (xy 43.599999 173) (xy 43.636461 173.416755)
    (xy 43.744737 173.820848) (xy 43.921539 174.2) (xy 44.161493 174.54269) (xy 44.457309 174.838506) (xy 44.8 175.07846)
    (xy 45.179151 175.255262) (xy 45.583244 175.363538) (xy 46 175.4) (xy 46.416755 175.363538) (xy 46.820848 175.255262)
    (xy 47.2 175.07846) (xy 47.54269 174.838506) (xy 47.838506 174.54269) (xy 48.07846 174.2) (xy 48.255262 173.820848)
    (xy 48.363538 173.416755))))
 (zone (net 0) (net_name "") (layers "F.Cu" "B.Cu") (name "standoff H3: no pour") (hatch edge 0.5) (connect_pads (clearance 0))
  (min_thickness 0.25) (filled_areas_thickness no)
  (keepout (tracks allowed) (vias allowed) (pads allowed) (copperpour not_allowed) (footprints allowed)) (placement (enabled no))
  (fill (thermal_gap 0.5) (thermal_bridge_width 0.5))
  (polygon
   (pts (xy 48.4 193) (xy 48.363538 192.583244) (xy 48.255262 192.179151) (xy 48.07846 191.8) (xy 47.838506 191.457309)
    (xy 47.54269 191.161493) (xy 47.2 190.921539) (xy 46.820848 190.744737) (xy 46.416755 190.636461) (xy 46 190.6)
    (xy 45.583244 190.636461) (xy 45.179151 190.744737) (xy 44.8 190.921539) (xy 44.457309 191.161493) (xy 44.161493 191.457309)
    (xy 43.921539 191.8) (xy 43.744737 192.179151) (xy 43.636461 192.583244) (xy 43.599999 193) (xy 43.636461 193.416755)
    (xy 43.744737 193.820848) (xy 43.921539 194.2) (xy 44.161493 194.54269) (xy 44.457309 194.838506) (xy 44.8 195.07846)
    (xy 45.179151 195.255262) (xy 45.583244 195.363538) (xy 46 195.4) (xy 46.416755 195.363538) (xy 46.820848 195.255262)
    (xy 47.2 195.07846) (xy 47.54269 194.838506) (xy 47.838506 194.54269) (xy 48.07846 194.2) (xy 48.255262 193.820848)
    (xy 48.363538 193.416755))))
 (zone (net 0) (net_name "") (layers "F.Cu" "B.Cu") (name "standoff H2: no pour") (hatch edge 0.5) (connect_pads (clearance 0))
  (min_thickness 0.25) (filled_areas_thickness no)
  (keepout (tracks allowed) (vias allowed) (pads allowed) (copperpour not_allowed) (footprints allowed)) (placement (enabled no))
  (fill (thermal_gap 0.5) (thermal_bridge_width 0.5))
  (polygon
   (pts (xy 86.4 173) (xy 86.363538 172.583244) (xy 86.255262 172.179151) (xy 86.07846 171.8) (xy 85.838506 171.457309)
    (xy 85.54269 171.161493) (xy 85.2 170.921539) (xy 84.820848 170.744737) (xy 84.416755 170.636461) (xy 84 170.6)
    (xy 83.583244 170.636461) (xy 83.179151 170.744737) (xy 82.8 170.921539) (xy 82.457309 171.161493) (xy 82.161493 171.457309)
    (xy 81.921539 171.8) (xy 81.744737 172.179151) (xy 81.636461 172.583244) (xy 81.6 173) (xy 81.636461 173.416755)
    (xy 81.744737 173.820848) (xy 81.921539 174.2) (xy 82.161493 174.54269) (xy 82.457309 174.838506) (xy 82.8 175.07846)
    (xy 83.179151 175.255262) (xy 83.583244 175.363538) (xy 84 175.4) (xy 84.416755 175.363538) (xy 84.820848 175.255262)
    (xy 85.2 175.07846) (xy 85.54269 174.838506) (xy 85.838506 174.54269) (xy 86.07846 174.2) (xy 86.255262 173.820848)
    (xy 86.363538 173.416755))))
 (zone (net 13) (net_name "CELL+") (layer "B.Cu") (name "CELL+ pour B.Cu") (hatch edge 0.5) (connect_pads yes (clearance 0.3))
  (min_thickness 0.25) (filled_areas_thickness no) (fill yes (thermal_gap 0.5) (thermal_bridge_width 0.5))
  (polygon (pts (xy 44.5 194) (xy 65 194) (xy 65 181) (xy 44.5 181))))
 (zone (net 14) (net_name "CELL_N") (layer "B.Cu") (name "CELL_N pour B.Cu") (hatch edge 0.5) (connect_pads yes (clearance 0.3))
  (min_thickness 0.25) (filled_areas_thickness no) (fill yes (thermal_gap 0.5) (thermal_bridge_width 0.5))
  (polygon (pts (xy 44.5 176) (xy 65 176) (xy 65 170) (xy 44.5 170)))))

